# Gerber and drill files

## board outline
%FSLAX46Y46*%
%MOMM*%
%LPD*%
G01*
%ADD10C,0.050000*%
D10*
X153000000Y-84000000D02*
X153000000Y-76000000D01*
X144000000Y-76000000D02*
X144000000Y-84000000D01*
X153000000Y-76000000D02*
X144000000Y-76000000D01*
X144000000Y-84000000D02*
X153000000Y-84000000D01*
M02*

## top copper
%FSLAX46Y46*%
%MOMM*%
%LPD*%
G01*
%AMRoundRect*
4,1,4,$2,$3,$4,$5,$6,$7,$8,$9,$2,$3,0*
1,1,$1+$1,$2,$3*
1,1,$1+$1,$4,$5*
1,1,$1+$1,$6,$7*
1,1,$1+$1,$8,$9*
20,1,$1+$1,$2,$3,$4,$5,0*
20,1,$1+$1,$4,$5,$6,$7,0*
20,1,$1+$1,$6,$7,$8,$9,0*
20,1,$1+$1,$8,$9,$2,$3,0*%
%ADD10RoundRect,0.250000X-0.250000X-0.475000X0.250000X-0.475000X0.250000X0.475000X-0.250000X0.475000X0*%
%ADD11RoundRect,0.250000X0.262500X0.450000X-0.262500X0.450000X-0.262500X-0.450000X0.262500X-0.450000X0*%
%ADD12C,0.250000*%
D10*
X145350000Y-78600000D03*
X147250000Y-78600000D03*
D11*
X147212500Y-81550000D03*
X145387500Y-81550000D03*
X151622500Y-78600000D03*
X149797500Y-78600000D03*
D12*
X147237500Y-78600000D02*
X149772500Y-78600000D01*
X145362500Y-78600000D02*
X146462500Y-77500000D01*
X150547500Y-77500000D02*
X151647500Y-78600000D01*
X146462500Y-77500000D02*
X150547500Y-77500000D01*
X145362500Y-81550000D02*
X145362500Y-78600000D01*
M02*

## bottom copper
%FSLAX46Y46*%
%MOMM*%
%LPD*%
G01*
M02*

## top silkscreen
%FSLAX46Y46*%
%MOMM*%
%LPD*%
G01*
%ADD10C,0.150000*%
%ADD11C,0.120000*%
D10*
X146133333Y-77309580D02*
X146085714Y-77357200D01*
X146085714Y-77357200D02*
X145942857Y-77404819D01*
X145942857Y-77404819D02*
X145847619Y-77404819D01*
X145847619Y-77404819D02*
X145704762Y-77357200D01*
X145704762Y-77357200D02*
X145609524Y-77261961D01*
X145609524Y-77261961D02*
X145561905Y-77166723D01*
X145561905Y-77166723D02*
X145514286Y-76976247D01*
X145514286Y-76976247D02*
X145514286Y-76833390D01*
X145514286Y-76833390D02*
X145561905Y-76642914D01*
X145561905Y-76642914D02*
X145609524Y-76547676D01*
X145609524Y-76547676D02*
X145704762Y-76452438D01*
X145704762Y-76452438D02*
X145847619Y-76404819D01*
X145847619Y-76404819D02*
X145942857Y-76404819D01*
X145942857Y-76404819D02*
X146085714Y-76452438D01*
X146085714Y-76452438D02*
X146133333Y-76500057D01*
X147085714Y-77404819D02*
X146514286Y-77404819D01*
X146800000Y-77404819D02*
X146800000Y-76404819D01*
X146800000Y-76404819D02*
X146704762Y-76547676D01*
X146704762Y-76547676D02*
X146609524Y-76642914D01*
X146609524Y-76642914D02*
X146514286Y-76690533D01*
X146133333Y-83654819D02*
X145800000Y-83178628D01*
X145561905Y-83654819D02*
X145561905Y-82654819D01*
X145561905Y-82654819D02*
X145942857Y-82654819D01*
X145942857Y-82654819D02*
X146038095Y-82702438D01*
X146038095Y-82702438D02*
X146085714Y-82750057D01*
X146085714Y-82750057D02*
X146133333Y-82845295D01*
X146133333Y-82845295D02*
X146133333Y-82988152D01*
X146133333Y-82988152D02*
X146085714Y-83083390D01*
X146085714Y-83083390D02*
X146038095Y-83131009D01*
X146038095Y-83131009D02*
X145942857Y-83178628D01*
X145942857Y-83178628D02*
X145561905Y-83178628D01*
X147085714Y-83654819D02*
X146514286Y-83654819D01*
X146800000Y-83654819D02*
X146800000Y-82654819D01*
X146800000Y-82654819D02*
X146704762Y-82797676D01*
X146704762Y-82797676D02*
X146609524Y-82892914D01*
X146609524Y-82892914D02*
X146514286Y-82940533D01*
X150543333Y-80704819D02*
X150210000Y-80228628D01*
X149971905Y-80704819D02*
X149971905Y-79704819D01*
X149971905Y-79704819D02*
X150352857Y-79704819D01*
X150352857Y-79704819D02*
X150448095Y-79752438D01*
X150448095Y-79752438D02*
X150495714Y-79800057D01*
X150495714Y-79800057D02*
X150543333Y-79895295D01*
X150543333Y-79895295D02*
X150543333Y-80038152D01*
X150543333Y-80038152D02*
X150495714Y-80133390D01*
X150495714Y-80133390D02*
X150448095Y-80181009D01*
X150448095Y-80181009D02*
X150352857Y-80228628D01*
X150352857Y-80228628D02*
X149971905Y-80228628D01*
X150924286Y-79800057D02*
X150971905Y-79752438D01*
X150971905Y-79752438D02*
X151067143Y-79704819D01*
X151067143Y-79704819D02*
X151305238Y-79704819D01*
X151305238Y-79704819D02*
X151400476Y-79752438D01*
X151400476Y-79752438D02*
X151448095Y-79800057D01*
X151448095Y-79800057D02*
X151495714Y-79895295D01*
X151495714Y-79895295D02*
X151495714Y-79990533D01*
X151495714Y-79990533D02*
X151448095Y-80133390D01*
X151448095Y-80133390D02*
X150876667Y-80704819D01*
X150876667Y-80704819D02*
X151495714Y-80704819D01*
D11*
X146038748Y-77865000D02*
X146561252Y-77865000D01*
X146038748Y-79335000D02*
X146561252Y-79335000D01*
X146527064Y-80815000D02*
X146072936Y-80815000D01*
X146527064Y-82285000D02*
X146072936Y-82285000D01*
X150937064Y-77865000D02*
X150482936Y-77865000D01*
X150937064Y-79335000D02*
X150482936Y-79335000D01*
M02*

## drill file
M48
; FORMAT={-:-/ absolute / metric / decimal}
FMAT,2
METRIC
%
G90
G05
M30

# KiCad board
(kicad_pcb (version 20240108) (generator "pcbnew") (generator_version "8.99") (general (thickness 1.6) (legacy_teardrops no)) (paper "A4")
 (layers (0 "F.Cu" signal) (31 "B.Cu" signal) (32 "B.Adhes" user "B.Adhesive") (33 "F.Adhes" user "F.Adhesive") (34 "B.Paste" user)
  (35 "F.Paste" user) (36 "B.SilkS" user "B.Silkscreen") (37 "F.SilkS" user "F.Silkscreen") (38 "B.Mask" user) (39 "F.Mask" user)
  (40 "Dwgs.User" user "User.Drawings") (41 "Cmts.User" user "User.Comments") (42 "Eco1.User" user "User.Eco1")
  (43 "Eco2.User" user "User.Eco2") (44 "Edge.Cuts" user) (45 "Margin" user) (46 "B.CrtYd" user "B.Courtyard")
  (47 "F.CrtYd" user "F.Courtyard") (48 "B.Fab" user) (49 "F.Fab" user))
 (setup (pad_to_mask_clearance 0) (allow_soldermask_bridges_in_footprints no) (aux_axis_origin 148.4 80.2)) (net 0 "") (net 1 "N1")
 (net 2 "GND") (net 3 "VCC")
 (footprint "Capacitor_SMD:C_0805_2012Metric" (layer "F.Cu") (at 146.3 78.6)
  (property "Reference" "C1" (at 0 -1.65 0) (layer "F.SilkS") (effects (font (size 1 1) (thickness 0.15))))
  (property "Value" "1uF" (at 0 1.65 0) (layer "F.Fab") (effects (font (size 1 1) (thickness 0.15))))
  (fp_line (start -0.261252 -0.735) (end 0.261252 -0.735) (stroke (width 0.12) (type solid)) (layer "F.SilkS"))
  (fp_line (start -0.261252 0.735) (end 0.261252 0.735) (stroke (width 0.12) (type solid)) (layer "F.SilkS"))
  (pad "1" smd roundrect (at -0.95 0) (size 1 1.45) (layers "F.Cu" "F.Paste" "F.Mask") (roundrect_rratio 0.25) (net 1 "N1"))
  (pad "2" smd roundrect (at 0.95 0) (size 1 1.45) (layers "F.Cu" "F.Paste" "F.Mask") (roundrect_rratio 0.25) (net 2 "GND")))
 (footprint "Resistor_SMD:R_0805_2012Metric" (layer "F.Cu") (at 146.3 81.55 180)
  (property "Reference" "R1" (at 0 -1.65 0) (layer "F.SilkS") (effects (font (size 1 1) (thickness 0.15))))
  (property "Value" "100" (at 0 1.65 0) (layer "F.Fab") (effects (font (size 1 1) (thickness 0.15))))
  (fp_line (start -0.227064 0.735) (end 0.227064 0.735) (stroke (width 0.12) (type solid)) (layer "F.SilkS"))
  (fp_line (start -0.227064 -0.735) (end 0.227064 -0.735) (stroke (width 0.12) (type solid)) (layer "F.SilkS"))
  (pad "1" smd roundrect (at -0.9125 0 180) (size 1.025 1.4) (layers "F.Cu" "F.Paste" "F.Mask") (roundrect_rratio 0.243902) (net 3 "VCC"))
  (pad "2" smd roundrect (at 0.9125 0 180) (size 1.025 1.4) (layers "F.Cu" "F.Paste" "F.Mask") (roundrect_rratio 0.243902) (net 1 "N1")))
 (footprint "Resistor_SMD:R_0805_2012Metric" (layer "F.Cu") (at 150.71 78.6 180)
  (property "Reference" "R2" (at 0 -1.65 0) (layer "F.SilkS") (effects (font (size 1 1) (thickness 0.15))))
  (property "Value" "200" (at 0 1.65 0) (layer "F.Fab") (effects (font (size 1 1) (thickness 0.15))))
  (fp_line (start -0.227064 0.735) (end 0.227064 0.735) (stroke (width 0.12) (type solid)) (layer "F.SilkS"))
  (fp_line (start -0.227064 -0.735) (end 0.227064 -0.735) (stroke (width 0.12) (type solid)) (layer "F.SilkS"))
  (pad "1" smd roundrect (at -0.9125 0 180) (size 1.025 1.4) (layers "F.Cu" "F.Paste" "F.Mask") (roundrect_rratio 0.243902) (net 1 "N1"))
  (pad "2" smd roundrect (at 0.9125 0 180) (size 1.025 1.4) (layers "F.Cu" "F.Paste" "F.Mask") (roundrect_rratio 0.243902) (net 2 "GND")))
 (gr_line (start 153 84) (end 153 76) (stroke (width 0.05) (type solid)) (layer "Edge.Cuts"))
 (gr_line (start 144 76) (end 144 84) (stroke (width 0.05) (type solid)) (layer "Edge.Cuts"))
 (gr_line (start 153 76) (end 144 76) (stroke (width 0.05) (type solid)) (layer "Edge.Cuts"))
 (gr_line (start 144 84) (end 153 84) (stroke (width 0.05) (type solid)) (layer "Edge.Cuts"))
 (segment (start 147.2375 78.6) (end 149.7725 78.6) (width 0.25) (layer "F.Cu") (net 2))
 (segment (start 145.3625 78.6) (end 146.4625 77.5) (width 0.25) (layer "F.Cu") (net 1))
 (segment (start 150.5475 77.5) (end 151.6475 78.6) (width 0.25) (layer "F.Cu") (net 1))
 (segment (start 146.4625 77.5) (end 150.5475 77.5) (width 0.25) (layer "F.Cu") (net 1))
 (segment (start 145.3625 81.55) (end 145.3625 78.6) (width 0.25) (layer "F.Cu") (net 1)))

